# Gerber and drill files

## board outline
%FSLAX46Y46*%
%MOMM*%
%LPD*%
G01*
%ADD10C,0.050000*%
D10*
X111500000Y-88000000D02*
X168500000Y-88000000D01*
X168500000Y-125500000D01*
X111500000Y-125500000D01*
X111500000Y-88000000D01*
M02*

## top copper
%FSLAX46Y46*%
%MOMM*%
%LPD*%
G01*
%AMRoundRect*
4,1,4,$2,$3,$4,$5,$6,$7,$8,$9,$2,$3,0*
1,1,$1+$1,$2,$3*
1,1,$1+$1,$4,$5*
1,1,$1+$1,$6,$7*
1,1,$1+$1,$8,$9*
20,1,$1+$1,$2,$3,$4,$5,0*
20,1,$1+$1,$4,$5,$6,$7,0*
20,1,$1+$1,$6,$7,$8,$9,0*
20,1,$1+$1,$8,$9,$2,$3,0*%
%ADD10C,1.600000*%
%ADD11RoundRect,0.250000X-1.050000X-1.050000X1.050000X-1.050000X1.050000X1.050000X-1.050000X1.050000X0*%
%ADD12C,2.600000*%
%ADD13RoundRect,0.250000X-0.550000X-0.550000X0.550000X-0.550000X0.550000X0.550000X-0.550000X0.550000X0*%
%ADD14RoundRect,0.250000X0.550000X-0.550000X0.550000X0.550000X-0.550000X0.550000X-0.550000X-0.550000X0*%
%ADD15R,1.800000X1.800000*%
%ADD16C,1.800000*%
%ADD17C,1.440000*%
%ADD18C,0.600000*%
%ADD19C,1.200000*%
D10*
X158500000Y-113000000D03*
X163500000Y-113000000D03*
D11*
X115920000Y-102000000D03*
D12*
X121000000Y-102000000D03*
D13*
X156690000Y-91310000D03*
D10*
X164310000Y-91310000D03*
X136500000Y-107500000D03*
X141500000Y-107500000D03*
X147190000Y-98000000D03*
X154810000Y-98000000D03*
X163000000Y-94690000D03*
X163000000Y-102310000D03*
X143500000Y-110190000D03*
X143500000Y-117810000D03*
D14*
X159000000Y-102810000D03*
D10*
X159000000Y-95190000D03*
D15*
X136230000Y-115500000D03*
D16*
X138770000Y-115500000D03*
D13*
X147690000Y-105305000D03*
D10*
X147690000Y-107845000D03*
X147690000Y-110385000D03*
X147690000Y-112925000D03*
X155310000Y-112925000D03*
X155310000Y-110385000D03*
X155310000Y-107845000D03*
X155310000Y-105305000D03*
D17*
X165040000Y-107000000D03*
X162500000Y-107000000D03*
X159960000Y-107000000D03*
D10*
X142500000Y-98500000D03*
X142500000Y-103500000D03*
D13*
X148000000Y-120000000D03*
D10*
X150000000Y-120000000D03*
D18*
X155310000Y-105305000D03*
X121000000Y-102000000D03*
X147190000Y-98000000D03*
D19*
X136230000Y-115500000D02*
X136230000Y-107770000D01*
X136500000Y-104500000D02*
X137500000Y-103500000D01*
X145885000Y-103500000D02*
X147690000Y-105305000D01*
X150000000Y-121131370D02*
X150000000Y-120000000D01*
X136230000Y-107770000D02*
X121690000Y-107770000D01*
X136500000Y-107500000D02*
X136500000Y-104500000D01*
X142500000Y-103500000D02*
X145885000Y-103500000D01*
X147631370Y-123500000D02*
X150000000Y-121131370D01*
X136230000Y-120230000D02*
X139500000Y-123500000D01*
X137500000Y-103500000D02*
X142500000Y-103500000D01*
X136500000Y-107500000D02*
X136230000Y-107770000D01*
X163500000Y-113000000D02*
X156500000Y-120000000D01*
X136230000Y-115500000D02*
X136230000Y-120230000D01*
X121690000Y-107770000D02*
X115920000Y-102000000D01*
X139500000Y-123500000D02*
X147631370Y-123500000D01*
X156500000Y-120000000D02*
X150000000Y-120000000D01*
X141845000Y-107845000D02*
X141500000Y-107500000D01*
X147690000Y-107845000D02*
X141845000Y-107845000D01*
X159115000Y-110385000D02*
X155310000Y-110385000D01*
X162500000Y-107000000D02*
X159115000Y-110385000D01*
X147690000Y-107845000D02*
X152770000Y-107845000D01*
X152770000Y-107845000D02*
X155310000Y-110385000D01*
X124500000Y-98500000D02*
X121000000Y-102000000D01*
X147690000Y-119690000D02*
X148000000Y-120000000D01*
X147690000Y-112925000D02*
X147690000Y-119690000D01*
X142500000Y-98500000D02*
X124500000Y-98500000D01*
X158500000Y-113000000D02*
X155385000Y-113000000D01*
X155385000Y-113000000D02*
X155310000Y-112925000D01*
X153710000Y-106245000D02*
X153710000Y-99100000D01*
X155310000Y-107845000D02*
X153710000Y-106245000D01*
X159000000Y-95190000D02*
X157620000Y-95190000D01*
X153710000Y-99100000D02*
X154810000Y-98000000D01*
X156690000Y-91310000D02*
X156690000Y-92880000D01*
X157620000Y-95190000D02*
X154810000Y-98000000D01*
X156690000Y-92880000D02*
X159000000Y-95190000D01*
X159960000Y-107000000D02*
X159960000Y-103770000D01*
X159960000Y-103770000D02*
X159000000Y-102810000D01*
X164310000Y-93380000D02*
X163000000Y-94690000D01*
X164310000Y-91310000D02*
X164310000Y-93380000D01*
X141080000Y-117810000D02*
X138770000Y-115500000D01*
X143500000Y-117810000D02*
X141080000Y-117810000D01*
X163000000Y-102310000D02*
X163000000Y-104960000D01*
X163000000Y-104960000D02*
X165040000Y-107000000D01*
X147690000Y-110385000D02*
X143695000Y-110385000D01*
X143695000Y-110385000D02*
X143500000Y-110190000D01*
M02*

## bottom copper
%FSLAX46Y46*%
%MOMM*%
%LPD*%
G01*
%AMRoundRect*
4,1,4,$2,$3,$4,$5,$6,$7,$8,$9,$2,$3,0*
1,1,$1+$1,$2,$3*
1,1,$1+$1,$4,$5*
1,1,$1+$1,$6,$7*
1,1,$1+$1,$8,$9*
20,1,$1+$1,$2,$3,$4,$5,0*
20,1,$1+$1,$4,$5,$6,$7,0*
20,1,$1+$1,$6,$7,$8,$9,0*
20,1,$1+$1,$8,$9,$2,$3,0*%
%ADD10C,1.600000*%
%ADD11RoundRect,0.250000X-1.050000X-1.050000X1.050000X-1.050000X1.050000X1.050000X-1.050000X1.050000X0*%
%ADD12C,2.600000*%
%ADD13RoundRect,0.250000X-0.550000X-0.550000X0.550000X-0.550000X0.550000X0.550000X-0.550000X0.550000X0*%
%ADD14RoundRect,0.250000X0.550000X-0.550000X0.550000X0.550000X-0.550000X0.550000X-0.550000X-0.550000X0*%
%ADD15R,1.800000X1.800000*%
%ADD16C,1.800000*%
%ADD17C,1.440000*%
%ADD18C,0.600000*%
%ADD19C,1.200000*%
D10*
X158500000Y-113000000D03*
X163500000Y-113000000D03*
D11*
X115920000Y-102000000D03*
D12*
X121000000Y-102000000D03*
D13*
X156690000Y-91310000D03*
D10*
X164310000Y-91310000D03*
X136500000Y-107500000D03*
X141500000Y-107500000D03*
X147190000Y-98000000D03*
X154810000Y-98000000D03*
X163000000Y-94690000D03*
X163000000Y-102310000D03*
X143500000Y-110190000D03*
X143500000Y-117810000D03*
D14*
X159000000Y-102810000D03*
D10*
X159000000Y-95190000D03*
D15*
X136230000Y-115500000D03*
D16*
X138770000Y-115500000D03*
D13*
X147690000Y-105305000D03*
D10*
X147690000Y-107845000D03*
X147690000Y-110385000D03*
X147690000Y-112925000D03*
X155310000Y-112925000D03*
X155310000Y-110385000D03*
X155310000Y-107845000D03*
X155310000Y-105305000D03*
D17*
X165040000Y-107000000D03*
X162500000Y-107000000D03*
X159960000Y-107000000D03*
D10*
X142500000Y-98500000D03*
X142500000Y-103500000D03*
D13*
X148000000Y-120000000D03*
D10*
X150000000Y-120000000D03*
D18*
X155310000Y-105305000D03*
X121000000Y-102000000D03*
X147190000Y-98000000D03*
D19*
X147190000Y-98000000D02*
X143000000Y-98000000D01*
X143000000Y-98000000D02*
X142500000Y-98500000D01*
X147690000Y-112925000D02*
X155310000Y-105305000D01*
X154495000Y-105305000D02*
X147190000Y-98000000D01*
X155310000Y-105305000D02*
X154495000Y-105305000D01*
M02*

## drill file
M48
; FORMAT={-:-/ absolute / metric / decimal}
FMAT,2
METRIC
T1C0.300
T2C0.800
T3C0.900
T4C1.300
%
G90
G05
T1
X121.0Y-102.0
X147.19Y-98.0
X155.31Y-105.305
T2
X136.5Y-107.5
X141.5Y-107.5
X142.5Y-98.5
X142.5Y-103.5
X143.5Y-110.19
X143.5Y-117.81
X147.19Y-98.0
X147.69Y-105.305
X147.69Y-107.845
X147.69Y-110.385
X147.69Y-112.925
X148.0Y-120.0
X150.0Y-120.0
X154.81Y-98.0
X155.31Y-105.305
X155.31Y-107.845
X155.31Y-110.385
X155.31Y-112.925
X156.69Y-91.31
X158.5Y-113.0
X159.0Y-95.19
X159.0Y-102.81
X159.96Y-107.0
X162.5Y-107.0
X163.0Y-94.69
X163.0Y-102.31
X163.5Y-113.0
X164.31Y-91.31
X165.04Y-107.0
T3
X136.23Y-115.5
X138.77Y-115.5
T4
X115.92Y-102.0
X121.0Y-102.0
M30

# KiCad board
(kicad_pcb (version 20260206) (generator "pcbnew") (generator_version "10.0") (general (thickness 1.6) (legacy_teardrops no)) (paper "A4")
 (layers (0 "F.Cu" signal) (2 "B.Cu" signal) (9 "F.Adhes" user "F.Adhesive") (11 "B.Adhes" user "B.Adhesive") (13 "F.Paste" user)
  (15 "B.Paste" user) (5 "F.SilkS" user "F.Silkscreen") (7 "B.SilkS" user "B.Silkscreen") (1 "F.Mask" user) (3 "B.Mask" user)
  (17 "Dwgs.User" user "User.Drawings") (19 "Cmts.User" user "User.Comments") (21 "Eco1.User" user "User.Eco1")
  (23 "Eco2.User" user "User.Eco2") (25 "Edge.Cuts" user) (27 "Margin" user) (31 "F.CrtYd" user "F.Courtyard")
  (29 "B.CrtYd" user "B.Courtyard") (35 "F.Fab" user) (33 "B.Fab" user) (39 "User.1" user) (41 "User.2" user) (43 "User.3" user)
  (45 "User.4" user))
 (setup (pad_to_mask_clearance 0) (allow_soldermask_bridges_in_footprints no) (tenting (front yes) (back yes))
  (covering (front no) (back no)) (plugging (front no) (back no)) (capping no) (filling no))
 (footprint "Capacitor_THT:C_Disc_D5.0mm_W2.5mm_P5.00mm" (layer "F.Cu") (at 158.5 113)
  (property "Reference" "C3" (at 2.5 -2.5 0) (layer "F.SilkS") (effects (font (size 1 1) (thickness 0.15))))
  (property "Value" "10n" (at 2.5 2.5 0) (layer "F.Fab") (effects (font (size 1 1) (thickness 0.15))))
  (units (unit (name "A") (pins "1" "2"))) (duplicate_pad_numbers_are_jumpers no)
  (pad "1" thru_hole circle (at 0 0) (size 1.6 1.6) (drill 0.8) (layers "*.Cu" "*.Mask") (remove_unused_layers no) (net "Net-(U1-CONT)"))
  (pad "2" thru_hole circle (at 5 0) (size 1.6 1.6) (drill 0.8) (layers "*.Cu" "*.Mask") (remove_unused_layers no) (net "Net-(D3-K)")))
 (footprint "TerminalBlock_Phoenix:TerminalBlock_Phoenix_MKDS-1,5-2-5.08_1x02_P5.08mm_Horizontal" (layer "F.Cu") (at 115.92 102)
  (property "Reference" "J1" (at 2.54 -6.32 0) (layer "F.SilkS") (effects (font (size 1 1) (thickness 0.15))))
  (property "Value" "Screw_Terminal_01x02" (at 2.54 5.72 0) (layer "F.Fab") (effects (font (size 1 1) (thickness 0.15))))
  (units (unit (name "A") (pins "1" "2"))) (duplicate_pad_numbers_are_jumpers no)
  (pad "1" thru_hole roundrect (at 0 0) (size 2.6 2.6) (drill 1.3) (layers "*.Cu" "*.Mask") (remove_unused_layers no)
   (roundrect_rratio 0.096154) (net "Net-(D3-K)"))
  (pad "2" thru_hole circle (at 5.08 0) (size 2.6 2.6) (drill 1.3) (layers "*.Cu" "*.Mask") (remove_unused_layers no) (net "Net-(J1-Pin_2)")))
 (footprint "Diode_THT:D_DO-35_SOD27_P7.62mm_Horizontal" (layer "F.Cu") (at 156.69 91.31)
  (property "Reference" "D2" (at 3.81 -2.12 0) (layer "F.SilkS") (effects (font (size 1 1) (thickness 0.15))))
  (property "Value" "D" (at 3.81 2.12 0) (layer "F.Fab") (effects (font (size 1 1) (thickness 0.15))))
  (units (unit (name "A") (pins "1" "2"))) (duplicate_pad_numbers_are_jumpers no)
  (pad "1" thru_hole roundrect (at 0 0) (size 1.6 1.6) (drill 0.8) (layers "*.Cu" "*.Mask") (remove_unused_layers no)
   (roundrect_rratio 0.15625) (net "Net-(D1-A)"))
  (pad "2" thru_hole circle (at 7.62 0) (size 1.6 1.6) (drill 0.8) (layers "*.Cu" "*.Mask") (remove_unused_layers no) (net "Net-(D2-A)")))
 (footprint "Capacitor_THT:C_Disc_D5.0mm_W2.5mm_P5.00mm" (layer "F.Cu") (at 136.5 107.5)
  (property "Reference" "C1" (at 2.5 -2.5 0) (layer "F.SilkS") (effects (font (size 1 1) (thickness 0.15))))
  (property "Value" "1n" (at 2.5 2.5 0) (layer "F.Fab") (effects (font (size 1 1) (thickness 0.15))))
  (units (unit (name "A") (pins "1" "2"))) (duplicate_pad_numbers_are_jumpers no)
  (pad "1" thru_hole circle (at 0 0) (size 1.6 1.6) (drill 0.8) (layers "*.Cu" "*.Mask") (remove_unused_layers no) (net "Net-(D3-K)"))
  (pad "2" thru_hole circle (at 5 0) (size 1.6 1.6) (drill 0.8) (layers "*.Cu" "*.Mask") (remove_unused_layers no) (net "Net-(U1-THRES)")))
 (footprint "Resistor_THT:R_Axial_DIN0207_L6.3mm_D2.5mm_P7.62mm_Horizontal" (layer "F.Cu") (at 147.19 98)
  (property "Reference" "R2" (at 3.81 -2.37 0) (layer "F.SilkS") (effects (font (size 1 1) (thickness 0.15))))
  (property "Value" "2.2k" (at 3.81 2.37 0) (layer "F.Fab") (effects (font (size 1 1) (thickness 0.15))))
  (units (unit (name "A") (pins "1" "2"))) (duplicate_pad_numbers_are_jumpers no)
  (pad "1" thru_hole circle (at 0 0) (size 1.6 1.6) (drill 0.8) (layers "*.Cu" "*.Mask") (remove_unused_layers no) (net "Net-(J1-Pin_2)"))
  (pad "2" thru_hole circle (at 7.62 0) (size 1.6 1.6) (drill 0.8) (layers "*.Cu" "*.Mask") (remove_unused_layers no) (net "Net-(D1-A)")))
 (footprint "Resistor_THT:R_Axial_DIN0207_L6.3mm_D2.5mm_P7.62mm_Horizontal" (layer "F.Cu") (at 163 94.69 -90)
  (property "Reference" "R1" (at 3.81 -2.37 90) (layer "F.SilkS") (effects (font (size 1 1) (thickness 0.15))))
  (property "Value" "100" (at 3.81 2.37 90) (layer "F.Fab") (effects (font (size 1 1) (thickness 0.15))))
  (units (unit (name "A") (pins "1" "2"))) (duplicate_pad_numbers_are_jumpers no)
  (pad "1" thru_hole circle (at 0 0 270) (size 1.6 1.6) (drill 0.8) (layers "*.Cu" "*.Mask") (remove_unused_layers no) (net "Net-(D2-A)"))
  (pad "2" thru_hole circle (at 7.62 0 270) (size 1.6 1.6) (drill 0.8) (layers "*.Cu" "*.Mask") (remove_unused_layers no)
   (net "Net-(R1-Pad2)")))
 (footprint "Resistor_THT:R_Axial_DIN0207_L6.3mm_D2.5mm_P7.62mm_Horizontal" (layer "F.Cu") (at 143.5 110.19 -90)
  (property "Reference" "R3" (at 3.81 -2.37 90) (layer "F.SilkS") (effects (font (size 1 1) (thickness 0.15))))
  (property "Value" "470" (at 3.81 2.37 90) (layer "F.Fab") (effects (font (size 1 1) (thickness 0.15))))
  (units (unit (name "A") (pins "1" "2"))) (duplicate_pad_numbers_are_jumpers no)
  (pad "1" thru_hole circle (at 0 0 270) (size 1.6 1.6) (drill 0.8) (layers "*.Cu" "*.Mask") (remove_unused_layers no) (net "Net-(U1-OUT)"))
  (pad "2" thru_hole circle (at 7.62 0 270) (size 1.6 1.6) (drill 0.8) (layers "*.Cu" "*.Mask") (remove_unused_layers no) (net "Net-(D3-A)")))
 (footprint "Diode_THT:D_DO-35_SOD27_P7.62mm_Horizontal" (layer "F.Cu") (at 159 102.81 90)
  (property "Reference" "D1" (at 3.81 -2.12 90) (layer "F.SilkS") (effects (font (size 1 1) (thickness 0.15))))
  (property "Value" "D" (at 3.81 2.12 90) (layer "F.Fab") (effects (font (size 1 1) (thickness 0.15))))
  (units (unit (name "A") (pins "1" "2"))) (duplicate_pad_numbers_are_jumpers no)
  (pad "1" thru_hole roundrect (at 0 0 90) (size 1.6 1.6) (drill 0.8) (layers "*.Cu" "*.Mask") (remove_unused_layers no)
   (roundrect_rratio 0.15625) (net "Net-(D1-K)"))
  (pad "2" thru_hole circle (at 7.62 0 90) (size 1.6 1.6) (drill 0.8) (layers "*.Cu" "*.Mask") (remove_unused_layers no) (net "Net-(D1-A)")))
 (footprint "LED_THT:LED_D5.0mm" (layer "F.Cu") (at 136.23 115.5)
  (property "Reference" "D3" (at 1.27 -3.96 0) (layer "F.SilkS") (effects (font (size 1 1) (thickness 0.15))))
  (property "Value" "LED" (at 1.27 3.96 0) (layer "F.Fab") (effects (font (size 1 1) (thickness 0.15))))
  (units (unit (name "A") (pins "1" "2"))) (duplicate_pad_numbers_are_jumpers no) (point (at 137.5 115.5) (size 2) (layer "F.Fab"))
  (pad "1" thru_hole rect (at 0 0) (size 1.8 1.8) (drill 0.9) (layers "*.Cu" "*.Mask") (remove_unused_layers no) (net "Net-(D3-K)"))
  (pad "2" thru_hole circle (at 2.54 0) (size 1.8 1.8) (drill 0.9) (layers "*.Cu" "*.Mask") (remove_unused_layers no) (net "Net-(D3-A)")))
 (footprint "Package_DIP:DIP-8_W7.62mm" (layer "F.Cu") (at 147.69 105.305)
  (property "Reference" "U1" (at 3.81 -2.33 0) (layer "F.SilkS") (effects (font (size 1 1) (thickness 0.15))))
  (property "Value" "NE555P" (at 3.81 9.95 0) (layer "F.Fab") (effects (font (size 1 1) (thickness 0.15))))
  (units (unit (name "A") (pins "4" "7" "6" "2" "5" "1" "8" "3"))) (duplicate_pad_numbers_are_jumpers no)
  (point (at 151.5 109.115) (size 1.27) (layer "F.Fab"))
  (pad "1" thru_hole roundrect (at 0 0) (size 1.6 1.6) (drill 0.8) (layers "*.Cu" "*.Mask") (remove_unused_layers no)
   (roundrect_rratio 0.15625) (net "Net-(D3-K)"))
  (pad "2" thru_hole circle (at 0 2.54) (size 1.6 1.6) (drill 0.8) (layers "*.Cu" "*.Mask") (remove_unused_layers no) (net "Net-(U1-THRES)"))
  (pad "3" thru_hole circle (at 0 5.08) (size 1.6 1.6) (drill 0.8) (layers "*.Cu" "*.Mask") (remove_unused_layers no) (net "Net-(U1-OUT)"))
  (pad "4" thru_hole circle (at 0 7.62) (size 1.6 1.6) (drill 0.8) (layers "*.Cu" "*.Mask") (remove_unused_layers no) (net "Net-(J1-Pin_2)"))
  (pad "5" thru_hole circle (at 7.62 7.62) (size 1.6 1.6) (drill 0.8) (layers "*.Cu" "*.Mask") (remove_unused_layers no)
   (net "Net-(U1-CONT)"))
  (pad "6" thru_hole circle (at 7.62 5.08) (size 1.6 1.6) (drill 0.8) (layers "*.Cu" "*.Mask") (remove_unused_layers no)
   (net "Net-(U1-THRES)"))
  (pad "7" thru_hole circle (at 7.62 2.54) (size 1.6 1.6) (drill 0.8) (layers "*.Cu" "*.Mask") (remove_unused_layers no) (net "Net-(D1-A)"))
  (pad "8" thru_hole circle (at 7.62 0) (size 1.6 1.6) (drill 0.8) (layers "*.Cu" "*.Mask") (remove_unused_layers no) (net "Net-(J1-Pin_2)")))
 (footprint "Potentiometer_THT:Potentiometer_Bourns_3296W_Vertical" (layer "F.Cu") (at 165.04 107)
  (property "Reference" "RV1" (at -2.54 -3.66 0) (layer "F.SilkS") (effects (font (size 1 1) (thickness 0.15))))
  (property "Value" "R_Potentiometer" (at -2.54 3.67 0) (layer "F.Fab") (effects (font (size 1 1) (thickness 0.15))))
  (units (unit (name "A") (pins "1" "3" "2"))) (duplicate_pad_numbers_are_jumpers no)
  (pad "1" thru_hole circle (at 0 0) (size 1.44 1.44) (drill 0.8) (layers "*.Cu" "*.Mask") (remove_unused_layers no) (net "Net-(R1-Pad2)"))
  (pad "2" thru_hole circle (at -2.54 0) (size 1.44 1.44) (drill 0.8) (layers "*.Cu" "*.Mask") (remove_unused_layers no)
   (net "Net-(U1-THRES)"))
  (pad "3" thru_hole circle (at -5.08 0) (size 1.44 1.44) (drill 0.8) (layers "*.Cu" "*.Mask") (remove_unused_layers no) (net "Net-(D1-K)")))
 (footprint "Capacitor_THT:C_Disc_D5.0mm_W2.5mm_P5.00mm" (layer "F.Cu") (at 142.5 98.5 -90)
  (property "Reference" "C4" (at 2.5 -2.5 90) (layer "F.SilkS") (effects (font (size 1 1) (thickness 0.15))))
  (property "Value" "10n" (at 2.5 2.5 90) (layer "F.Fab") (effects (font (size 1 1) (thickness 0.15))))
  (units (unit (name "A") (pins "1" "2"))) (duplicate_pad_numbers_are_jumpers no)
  (pad "1" thru_hole circle (at 0 0 270) (size 1.6 1.6) (drill 0.8) (layers "*.Cu" "*.Mask") (remove_unused_layers no)
   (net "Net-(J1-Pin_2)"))
  (pad "2" thru_hole circle (at 5 0 270) (size 1.6 1.6) (drill 0.8) (layers "*.Cu" "*.Mask") (remove_unused_layers no) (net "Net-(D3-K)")))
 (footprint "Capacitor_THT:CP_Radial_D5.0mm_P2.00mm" (layer "F.Cu") (at 148 120)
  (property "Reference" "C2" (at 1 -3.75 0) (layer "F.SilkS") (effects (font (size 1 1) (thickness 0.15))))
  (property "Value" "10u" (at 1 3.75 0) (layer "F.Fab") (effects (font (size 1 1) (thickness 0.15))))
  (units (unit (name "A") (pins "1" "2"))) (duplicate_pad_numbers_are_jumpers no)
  (pad "1" thru_hole roundrect (at 0 0) (size 1.6 1.6) (drill 0.8) (layers "*.Cu" "*.Mask") (remove_unused_layers no)
   (roundrect_rratio 0.15625) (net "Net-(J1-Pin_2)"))
  (pad "2" thru_hole circle (at 2 0) (size 1.6 1.6) (drill 0.8) (layers "*.Cu" "*.Mask") (remove_unused_layers no) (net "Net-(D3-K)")))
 (gr_rect (start 111.5 88) (end 168.5 125.5) (stroke (width 0.05) (type default)) (fill no) (layer "Edge.Cuts"))
 (segment (start 136.23 115.5) (end 136.23 107.77) (width 1.2) (layer "F.Cu") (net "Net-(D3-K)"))
 (segment (start 136.5 104.5) (end 137.5 103.5) (width 1.2) (layer "F.Cu") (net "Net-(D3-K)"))
 (segment (start 145.885 103.5) (end 147.69 105.305) (width 1.2) (layer "F.Cu") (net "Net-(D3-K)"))
 (segment (start 150 121.13137) (end 150 120) (width 1.2) (layer "F.Cu") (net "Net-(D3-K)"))
 (segment (start 136.23 107.77) (end 121.69 107.77) (width 1.2) (layer "F.Cu") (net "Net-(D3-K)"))
 (segment (start 136.5 107.5) (end 136.5 104.5) (width 1.2) (layer "F.Cu") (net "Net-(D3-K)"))
 (segment (start 142.5 103.5) (end 145.885 103.5) (width 1.2) (layer "F.Cu") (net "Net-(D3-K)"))
 (segment (start 147.63137 123.5) (end 150 121.13137) (width 1.2) (layer "F.Cu") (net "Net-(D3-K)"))
 (segment (start 136.23 120.23) (end 139.5 123.5) (width 1.2) (layer "F.Cu") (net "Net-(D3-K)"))
 (segment (start 137.5 103.5) (end 142.5 103.5) (width 1.2) (layer "F.Cu") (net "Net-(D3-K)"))
 (segment (start 136.5 107.5) (end 136.23 107.77) (width 1.2) (layer "F.Cu") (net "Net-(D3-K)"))
 (segment (start 163.5 113) (end 156.5 120) (width 1.2) (layer "F.Cu") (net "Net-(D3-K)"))
 (segment (start 136.23 115.5) (end 136.23 120.23) (width 1.2) (layer "F.Cu") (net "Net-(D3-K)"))
 (segment (start 121.69 107.77) (end 115.92 102) (width 1.2) (layer "F.Cu") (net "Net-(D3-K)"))
 (segment (start 139.5 123.5) (end 147.63137 123.5) (width 1.2) (layer "F.Cu") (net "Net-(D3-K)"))
 (segment (start 156.5 120) (end 150 120) (width 1.2) (layer "F.Cu") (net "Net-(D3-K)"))
 (segment (start 141.845 107.845) (end 141.5 107.5) (width 1.2) (layer "F.Cu") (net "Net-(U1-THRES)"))
 (segment (start 147.69 107.845) (end 141.845 107.845) (width 1.2) (layer "F.Cu") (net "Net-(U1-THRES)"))
 (segment (start 159.115 110.385) (end 155.31 110.385) (width 1.2) (layer "F.Cu") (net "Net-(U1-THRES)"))
 (segment (start 162.5 107) (end 159.115 110.385) (width 1.2) (layer "F.Cu") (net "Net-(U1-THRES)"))
 (segment (start 147.69 107.845) (end 152.77 107.845) (width 1.2) (layer "F.Cu") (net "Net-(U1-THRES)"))
 (segment (start 152.77 107.845) (end 155.31 110.385) (width 1.2) (layer "F.Cu") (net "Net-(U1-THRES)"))
 (segment (start 124.5 98.5) (end 121 102) (width 1.2) (layer "F.Cu") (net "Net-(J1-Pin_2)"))
 (segment (start 147.69 119.69) (end 148 120) (width 1.2) (layer "F.Cu") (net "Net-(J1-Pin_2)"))
 (segment (start 147.69 112.925) (end 147.69 119.69) (width 1.2) (layer "F.Cu") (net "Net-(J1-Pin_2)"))
 (segment (start 142.5 98.5) (end 124.5 98.5) (width 1.2) (layer "F.Cu") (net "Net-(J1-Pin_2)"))
 (via (at 155.31 105.305) (size 0.6) (drill 0.3) (layers "F.Cu" "B.Cu") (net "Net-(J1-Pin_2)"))
 (via (at 121 102) (size 0.6) (drill 0.3) (layers "F.Cu" "B.Cu") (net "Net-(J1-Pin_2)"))
 (via (at 147.19 98) (size 0.6) (drill 0.3) (layers "F.Cu" "B.Cu") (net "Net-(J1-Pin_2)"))
 (segment (start 147.19 98) (end 143 98) (width 1.2) (layer "B.Cu") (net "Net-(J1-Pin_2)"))
 (segment (start 143 98) (end 142.5 98.5) (width 1.2) (layer "B.Cu") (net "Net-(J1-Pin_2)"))
 (segment (start 147.69 112.925) (end 155.31 105.305) (width 1.2) (layer "B.Cu") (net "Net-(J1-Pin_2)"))
 (segment (start 154.495 105.305) (end 147.19 98) (width 1.2) (layer "B.Cu") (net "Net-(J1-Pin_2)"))
 (segment (start 155.31 105.305) (end 154.495 105.305) (width 1.2) (layer "B.Cu") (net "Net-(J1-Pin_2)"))
 (segment (start 158.5 113) (end 155.385 113) (width 1.2) (layer "F.Cu") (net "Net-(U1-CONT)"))
 (segment (start 155.385 113) (end 155.31 112.925) (width 1.2) (layer "F.Cu") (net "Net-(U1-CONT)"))
 (segment (start 153.71 106.245) (end 153.71 99.1) (width 1.2) (layer "F.Cu") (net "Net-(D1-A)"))
 (segment (start 155.31 107.845) (end 153.71 106.245) (width 1.2) (layer "F.Cu") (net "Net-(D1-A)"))
 (segment (start 159 95.19) (end 157.62 95.19) (width 1.2) (layer "F.Cu") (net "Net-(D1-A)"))
 (segment (start 153.71 99.1) (end 154.81 98) (width 1.2) (layer "F.Cu") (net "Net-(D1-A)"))
 (segment (start 156.69 91.31) (end 156.69 92.88) (width 1.2) (layer "F.Cu") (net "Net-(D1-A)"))
 (segment (start 157.62 95.19) (end 154.81 98) (width 1.2) (layer "F.Cu") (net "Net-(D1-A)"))
 (segment (start 156.69 92.88) (end 159 95.19) (width 1.2) (layer "F.Cu") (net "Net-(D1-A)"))
 (segment (start 159.96 107) (end 159.96 103.77) (width 1.2) (layer "F.Cu") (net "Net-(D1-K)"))
 (segment (start 159.96 103.77) (end 159 102.81) (width 1.2) (layer "F.Cu") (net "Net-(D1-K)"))
 (segment (start 164.31 93.38) (end 163 94.69) (width 1.2) (layer "F.Cu") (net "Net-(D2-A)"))
 (segment (start 164.31 91.31) (end 164.31 93.38) (width 1.2) (layer "F.Cu") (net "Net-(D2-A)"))
 (segment (start 141.08 117.81) (end 138.77 115.5) (width 1.2) (layer "F.Cu") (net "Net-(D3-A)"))
 (segment (start 143.5 117.81) (end 141.08 117.81) (width 1.2) (layer "F.Cu") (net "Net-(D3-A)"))
 (segment (start 163 102.31) (end 163 104.96) (width 1.2) (layer "F.Cu") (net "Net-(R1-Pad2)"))
 (segment (start 163 104.96) (end 165.04 107) (width 1.2) (layer "F.Cu") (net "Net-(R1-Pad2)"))
 (segment (start 147.69 110.385) (end 143.695 110.385) (width 1.2) (layer "F.Cu") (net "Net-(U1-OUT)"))
 (segment (start 143.695 110.385) (end 143.5 110.19) (width 1.2) (layer "F.Cu") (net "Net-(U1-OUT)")))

